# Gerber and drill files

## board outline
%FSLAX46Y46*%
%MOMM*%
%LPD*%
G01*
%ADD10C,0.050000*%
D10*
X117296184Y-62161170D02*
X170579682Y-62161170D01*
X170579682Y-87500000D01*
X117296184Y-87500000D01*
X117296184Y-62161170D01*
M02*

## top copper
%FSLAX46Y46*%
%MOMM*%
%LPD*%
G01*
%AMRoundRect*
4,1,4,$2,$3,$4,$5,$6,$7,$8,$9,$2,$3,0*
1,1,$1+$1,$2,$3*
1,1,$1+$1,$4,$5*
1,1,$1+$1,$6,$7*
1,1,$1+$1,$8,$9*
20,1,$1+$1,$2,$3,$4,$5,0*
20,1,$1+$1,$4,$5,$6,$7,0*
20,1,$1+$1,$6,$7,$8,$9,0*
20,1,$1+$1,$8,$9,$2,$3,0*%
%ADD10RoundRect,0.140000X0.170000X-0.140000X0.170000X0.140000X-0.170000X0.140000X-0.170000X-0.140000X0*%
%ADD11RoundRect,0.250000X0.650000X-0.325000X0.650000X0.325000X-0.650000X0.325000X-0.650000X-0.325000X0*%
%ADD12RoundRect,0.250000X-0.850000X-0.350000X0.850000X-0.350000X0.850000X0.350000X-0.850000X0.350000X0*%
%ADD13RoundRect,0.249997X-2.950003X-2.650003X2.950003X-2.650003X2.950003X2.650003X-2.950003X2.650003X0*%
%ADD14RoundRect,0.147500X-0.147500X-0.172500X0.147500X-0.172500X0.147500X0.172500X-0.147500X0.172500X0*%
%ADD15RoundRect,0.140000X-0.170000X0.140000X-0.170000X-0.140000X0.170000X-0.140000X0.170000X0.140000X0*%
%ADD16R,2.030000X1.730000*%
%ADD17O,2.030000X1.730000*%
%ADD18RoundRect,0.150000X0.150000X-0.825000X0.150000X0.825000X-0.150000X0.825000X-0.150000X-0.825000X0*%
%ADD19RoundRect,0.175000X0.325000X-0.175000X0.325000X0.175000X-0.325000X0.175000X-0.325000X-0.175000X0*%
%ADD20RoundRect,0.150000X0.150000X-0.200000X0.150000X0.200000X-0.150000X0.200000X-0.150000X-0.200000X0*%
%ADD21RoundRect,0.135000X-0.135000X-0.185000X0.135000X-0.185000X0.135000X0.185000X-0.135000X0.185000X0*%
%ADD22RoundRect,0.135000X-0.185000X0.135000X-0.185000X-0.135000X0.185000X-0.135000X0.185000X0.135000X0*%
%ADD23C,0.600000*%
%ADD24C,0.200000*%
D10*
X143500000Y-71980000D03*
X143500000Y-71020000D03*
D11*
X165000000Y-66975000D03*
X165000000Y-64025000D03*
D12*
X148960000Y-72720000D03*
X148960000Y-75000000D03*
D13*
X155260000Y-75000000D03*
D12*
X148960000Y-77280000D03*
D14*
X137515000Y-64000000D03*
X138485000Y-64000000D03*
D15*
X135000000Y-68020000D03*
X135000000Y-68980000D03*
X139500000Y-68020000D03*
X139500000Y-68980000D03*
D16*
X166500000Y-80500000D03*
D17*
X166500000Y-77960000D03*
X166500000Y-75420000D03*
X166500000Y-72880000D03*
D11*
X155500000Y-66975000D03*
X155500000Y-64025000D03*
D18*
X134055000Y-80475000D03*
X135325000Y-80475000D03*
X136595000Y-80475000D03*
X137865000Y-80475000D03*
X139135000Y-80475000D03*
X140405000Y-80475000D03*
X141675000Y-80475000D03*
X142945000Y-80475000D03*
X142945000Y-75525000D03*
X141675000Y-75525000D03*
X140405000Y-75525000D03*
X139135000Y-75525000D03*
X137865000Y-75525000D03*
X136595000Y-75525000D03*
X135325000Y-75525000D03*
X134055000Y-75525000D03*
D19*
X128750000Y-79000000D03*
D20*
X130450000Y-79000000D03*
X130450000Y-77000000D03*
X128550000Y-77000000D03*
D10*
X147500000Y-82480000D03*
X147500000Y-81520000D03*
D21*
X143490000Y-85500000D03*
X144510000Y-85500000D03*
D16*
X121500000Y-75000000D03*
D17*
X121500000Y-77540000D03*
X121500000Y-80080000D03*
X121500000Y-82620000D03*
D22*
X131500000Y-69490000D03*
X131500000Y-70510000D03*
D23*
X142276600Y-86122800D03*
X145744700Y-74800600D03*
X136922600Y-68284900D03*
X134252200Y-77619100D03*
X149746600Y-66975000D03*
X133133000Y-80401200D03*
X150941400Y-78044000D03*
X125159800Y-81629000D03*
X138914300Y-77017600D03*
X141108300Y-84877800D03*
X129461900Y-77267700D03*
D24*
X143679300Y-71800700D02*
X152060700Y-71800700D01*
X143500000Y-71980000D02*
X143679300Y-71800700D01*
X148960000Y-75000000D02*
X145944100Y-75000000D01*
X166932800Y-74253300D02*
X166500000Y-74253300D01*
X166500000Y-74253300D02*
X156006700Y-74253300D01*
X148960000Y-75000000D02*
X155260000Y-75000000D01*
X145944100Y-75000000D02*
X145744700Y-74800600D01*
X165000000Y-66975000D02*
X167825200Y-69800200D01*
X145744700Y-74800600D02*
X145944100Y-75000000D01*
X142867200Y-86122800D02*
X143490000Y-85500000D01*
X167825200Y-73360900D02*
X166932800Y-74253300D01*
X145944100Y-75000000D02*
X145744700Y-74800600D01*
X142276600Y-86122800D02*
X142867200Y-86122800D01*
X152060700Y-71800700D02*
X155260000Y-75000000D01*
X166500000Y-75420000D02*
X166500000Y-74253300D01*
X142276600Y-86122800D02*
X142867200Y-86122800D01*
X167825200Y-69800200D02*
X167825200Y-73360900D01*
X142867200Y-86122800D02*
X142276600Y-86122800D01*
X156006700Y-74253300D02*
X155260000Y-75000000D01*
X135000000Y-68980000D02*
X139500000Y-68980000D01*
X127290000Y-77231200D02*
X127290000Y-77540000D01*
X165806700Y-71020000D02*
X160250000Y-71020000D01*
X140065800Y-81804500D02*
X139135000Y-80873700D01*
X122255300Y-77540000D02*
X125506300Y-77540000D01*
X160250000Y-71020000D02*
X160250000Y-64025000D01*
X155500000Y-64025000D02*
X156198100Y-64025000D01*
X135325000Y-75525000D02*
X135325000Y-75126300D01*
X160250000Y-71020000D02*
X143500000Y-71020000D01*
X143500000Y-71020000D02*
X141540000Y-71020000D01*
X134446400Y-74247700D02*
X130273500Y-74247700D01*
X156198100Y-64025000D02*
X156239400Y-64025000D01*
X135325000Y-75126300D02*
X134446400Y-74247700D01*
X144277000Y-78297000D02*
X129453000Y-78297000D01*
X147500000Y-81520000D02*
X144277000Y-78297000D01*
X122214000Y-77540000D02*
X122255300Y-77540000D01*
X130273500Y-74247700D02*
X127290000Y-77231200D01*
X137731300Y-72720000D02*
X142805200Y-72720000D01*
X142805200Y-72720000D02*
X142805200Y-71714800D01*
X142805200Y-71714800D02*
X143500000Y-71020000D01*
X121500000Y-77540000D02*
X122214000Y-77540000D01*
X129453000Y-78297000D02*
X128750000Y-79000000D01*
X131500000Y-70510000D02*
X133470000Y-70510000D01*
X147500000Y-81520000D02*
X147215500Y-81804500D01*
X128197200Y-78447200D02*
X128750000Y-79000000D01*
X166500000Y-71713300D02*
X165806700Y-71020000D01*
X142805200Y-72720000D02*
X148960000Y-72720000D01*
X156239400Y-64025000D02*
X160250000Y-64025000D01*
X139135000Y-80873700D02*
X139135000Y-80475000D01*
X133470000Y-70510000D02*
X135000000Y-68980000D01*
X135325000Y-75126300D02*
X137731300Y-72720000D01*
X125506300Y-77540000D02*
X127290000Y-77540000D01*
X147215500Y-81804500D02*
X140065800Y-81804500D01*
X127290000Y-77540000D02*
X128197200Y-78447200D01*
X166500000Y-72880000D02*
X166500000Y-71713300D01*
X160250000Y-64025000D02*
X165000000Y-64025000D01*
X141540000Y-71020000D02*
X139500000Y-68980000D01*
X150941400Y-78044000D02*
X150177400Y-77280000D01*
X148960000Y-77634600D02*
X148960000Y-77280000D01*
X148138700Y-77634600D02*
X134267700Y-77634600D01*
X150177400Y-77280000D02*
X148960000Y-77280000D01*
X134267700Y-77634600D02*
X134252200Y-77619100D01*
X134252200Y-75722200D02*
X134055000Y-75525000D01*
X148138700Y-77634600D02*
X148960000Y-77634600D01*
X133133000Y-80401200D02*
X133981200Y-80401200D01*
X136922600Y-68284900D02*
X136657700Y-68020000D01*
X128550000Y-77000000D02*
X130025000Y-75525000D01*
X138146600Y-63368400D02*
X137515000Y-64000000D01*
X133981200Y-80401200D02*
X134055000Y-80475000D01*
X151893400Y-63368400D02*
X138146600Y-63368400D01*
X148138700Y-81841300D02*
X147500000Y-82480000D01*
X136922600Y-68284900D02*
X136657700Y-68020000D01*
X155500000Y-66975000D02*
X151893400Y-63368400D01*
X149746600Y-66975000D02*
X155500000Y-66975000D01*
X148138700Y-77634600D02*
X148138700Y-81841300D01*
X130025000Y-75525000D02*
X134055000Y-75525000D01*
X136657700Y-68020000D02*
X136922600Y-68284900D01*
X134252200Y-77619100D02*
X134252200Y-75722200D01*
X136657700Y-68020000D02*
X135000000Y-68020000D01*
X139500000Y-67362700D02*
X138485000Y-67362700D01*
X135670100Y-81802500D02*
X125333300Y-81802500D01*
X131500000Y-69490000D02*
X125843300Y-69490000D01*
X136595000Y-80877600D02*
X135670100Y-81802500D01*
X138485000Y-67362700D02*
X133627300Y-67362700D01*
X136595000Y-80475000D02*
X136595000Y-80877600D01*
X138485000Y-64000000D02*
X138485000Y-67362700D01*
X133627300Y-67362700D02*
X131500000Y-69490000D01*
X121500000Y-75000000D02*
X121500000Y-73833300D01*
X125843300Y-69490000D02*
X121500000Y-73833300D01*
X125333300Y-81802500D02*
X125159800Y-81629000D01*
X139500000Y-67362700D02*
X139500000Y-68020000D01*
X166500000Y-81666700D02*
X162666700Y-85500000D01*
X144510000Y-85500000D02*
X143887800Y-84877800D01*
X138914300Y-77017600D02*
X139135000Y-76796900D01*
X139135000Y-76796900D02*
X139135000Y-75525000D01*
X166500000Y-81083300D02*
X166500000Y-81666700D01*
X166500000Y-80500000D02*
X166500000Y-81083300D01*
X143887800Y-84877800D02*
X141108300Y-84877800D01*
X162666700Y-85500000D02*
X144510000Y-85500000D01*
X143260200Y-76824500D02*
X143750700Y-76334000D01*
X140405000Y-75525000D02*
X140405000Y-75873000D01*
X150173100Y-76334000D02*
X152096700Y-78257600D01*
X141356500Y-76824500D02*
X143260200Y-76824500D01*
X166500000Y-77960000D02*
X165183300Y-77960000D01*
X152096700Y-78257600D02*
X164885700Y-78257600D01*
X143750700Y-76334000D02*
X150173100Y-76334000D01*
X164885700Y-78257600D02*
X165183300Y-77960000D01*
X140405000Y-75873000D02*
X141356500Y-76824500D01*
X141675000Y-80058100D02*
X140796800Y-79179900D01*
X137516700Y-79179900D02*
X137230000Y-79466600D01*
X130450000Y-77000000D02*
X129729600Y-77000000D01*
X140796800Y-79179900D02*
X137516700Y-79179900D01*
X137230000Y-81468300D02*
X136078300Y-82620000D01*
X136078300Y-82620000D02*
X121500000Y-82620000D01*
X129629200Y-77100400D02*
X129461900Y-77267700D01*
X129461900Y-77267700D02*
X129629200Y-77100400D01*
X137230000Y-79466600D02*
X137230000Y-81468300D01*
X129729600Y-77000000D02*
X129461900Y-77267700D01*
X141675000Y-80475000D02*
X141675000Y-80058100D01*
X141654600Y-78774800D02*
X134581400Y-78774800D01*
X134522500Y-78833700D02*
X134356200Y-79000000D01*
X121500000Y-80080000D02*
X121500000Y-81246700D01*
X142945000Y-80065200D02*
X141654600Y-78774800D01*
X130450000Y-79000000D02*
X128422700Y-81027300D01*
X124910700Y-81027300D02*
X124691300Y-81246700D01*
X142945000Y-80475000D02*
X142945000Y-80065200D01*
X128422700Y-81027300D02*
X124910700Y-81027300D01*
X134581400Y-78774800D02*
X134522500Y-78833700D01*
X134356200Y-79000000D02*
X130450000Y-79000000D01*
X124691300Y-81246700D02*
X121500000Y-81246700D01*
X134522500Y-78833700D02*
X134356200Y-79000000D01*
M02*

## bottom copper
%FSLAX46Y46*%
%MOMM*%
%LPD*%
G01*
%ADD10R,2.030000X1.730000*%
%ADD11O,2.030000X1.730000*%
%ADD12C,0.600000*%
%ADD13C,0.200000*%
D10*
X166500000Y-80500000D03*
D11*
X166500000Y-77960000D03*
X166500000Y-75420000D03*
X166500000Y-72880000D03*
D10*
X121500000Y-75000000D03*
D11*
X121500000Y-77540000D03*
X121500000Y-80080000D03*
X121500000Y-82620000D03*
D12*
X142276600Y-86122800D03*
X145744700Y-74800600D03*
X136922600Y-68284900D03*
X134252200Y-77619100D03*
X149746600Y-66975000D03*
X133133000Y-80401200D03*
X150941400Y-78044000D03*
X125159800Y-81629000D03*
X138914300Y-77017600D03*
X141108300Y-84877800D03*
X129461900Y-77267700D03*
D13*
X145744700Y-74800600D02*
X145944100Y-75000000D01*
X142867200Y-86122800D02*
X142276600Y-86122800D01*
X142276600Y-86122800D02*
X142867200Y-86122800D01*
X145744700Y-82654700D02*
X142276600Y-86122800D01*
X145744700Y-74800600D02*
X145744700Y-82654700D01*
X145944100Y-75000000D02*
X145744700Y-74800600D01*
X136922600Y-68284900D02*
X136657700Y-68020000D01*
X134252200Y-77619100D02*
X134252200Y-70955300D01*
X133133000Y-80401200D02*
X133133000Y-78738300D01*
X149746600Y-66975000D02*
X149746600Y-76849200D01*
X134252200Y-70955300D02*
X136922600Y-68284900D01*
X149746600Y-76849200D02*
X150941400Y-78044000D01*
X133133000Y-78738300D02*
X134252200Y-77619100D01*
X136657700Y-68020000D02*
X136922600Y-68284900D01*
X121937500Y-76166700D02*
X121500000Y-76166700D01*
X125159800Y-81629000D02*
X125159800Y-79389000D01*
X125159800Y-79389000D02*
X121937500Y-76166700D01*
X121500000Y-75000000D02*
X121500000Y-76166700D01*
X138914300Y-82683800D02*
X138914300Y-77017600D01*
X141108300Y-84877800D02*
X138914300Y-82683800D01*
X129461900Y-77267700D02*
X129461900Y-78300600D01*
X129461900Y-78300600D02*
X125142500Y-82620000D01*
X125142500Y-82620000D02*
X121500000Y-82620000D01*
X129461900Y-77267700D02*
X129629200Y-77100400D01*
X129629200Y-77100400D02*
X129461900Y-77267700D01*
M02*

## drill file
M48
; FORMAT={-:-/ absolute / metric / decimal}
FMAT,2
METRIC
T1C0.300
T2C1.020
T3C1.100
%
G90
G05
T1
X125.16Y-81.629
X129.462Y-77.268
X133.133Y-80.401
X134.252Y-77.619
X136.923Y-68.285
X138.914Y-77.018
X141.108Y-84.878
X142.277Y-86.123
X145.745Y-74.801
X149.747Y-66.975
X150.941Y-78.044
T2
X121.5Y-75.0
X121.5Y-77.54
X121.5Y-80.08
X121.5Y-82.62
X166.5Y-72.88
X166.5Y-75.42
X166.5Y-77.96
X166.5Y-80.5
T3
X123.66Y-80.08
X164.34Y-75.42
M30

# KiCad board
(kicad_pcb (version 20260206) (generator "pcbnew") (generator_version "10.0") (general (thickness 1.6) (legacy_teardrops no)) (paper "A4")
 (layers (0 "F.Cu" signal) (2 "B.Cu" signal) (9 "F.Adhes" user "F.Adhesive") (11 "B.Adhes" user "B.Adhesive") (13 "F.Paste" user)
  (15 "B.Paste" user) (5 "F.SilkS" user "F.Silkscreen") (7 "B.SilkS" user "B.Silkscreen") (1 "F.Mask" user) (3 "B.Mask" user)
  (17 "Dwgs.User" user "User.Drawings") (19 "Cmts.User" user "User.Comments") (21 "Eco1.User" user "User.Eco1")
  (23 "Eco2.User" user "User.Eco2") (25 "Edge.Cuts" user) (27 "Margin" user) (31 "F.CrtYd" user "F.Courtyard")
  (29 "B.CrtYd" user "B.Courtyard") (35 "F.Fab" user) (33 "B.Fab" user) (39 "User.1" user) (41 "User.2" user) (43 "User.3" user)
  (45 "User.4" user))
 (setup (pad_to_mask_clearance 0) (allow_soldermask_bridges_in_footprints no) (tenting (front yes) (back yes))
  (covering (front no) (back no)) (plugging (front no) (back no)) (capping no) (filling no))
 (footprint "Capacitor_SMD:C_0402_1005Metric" (layer "F.Cu") (at 143.5 71.5 90)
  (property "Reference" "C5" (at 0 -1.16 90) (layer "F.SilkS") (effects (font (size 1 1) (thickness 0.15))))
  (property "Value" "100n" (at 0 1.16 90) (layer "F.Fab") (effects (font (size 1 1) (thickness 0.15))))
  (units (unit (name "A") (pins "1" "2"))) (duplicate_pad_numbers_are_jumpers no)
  (pad "1" smd roundrect (at -0.48 0 90) (size 0.56 0.62) (layers "F.Cu" "F.Mask" "F.Paste") (roundrect_rratio 0.25) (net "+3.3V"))
  (pad "2" smd roundrect (at 0.48 0 90) (size 0.56 0.62) (layers "F.Cu" "F.Mask" "F.Paste") (roundrect_rratio 0.25) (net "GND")))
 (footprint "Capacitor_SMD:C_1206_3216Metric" (layer "F.Cu") (at 165 65.5 90)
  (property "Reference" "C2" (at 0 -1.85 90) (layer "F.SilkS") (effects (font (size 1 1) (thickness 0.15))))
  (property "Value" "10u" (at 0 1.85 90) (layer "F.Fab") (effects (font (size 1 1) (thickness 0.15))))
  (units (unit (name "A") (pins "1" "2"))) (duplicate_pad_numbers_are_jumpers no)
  (pad "1" smd roundrect (at -1.475 0 90) (size 1.15 1.8) (layers "F.Cu" "F.Mask" "F.Paste") (roundrect_rratio 0.217391) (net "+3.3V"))
  (pad "2" smd roundrect (at 1.475 0 90) (size 1.15 1.8) (layers "F.Cu" "F.Mask" "F.Paste") (roundrect_rratio 0.217391) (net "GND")))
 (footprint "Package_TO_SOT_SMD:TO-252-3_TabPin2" (layer "F.Cu") (at 154 75)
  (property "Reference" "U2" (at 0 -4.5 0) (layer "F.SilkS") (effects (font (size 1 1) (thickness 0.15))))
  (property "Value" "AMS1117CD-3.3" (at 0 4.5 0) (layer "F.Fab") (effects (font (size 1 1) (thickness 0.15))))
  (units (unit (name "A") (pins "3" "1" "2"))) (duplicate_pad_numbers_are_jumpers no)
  (pad "" smd roundrect (at -0.415 -1.525) (size 3.05 2.75) (layers "F.Paste") (roundrect_rratio 0.090909))
  (pad "" smd roundrect (at -0.415 1.525) (size 3.05 2.75) (layers "F.Paste") (roundrect_rratio 0.090909))
  (pad "" smd roundrect (at 2.935 -1.525) (size 3.05 2.75) (layers "F.Paste") (roundrect_rratio 0.090909))
  (pad "" smd roundrect (at 2.935 1.525) (size 3.05 2.75) (layers "F.Paste") (roundrect_rratio 0.090909))
  (pad "1" smd roundrect (at -5.04 -2.28) (size 2.2 1.2) (layers "F.Cu" "F.Mask" "F.Paste") (roundrect_rratio 0.208333) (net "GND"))
  (pad "2" smd roundrect (at -5.04 0) (size 2.2 1.2) (layers "F.Cu" "F.Mask" "F.Paste") (roundrect_rratio 0.208333) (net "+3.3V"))
  (pad "2" smd roundrect (at 1.26 0) (size 6.4 5.8) (layers "F.Cu" "F.Mask") (roundrect_rratio 0.043103) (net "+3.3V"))
  (pad "3" smd roundrect (at -5.04 2.28) (size 2.2 1.2) (layers "F.Cu" "F.Mask" "F.Paste") (roundrect_rratio 0.208333) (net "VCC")))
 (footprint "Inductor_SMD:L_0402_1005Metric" (layer "F.Cu") (at 138 64)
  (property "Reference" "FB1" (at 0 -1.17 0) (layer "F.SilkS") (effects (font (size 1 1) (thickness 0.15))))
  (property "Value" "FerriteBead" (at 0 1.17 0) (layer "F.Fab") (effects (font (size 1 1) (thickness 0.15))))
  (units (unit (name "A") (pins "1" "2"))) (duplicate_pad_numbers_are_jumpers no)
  (pad "1" smd roundrect (at -0.485 0) (size 0.59 0.64) (layers "F.Cu" "F.Mask" "F.Paste") (roundrect_rratio 0.25) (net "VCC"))
  (pad "2" smd roundrect (at 0.485 0) (size 0.59 0.64) (layers "F.Cu" "F.Mask" "F.Paste") (roundrect_rratio 0.25) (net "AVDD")))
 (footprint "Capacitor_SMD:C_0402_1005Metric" (layer "F.Cu") (at 135 68.5 -90)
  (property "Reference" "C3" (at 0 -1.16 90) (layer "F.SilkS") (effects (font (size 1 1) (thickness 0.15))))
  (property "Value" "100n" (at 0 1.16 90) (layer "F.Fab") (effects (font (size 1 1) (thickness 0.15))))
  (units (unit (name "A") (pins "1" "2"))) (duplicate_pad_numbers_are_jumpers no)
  (pad "1" smd roundrect (at -0.48 0 270) (size 0.56 0.62) (layers "F.Cu" "F.Mask" "F.Paste") (roundrect_rratio 0.25) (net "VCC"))
  (pad "2" smd roundrect (at 0.48 0 270) (size 0.56 0.62) (layers "F.Cu" "F.Mask" "F.Paste") (roundrect_rratio 0.25) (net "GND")))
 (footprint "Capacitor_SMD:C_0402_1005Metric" (layer "F.Cu") (at 139.5 68.5 -90)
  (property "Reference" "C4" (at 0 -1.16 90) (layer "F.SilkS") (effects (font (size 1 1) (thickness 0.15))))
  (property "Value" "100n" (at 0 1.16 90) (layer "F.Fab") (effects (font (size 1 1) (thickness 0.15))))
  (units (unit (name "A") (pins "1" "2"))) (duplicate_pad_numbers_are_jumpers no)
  (pad "1" smd roundrect (at -0.48 0 270) (size 0.56 0.62) (layers "F.Cu" "F.Mask" "F.Paste") (roundrect_rratio 0.25) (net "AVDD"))
  (pad "2" smd roundrect (at 0.48 0 270) (size 0.56 0.62) (layers "F.Cu" "F.Mask" "F.Paste") (roundrect_rratio 0.25) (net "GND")))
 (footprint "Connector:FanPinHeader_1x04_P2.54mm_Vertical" (layer "F.Cu") (at 166.5 80.5 90)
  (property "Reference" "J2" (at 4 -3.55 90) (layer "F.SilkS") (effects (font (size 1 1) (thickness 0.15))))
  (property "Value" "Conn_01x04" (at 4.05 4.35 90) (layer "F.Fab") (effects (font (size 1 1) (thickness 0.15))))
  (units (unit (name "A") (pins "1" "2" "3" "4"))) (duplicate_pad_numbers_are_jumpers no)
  (pad "" np_thru_hole circle (at 5.08 -2.16 180) (size 1.1 1.1) (drill 1.1) (layers "*.Cu" "*.Mask"))
  (pad "1" thru_hole rect (at 0 0 180) (size 2.03 1.73) (drill 1.02) (layers "*.Cu" "*.Mask") (remove_unused_layers no) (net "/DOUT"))
  (pad "2" thru_hole oval (at 2.54 0 180) (size 2.03 1.73) (drill 1.02) (layers "*.Cu" "*.Mask") (remove_unused_layers no) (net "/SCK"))
  (pad "3" thru_hole oval (at 5.08 0 180) (size 2.03 1.73) (drill 1.02) (layers "*.Cu" "*.Mask") (remove_unused_layers no) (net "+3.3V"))
  (pad "4" thru_hole oval (at 7.62 0 180) (size 2.03 1.73) (drill 1.02) (layers "*.Cu" "*.Mask") (remove_unused_layers no) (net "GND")))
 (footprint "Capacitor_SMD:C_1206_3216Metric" (layer "F.Cu") (at 155.5 65.5 90)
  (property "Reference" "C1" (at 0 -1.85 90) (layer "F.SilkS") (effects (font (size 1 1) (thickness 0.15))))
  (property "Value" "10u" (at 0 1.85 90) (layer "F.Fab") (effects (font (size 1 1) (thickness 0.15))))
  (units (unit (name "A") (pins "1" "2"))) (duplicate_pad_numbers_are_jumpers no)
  (pad "1" smd roundrect (at -1.475 0 90) (size 1.15 1.8) (layers "F.Cu" "F.Mask" "F.Paste") (roundrect_rratio 0.217391) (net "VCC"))
  (pad "2" smd roundrect (at 1.475 0 90) (size 1.15 1.8) (layers "F.Cu" "F.Mask" "F.Paste") (roundrect_rratio 0.217391) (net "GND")))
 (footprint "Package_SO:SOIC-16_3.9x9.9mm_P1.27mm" (layer "F.Cu") (at 138.5 78 90)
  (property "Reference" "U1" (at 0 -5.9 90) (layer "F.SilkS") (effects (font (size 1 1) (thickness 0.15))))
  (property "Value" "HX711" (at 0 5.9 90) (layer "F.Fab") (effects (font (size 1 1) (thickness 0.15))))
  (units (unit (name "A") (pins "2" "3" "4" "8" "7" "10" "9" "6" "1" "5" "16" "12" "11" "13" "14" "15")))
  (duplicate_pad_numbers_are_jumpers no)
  (pad "1" smd roundrect (at -2.475 -4.445 90) (size 1.95 0.6) (layers "F.Cu" "F.Mask" "F.Paste") (roundrect_rratio 0.25) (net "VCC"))
  (pad "2" smd roundrect (at -2.475 -3.175 90) (size 1.95 0.6) (layers "F.Cu" "F.Mask" "F.Paste") (roundrect_rratio 0.25)
   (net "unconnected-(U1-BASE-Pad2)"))
  (pad "3" smd roundrect (at -2.475 -1.905 90) (size 1.95 0.6) (layers "F.Cu" "F.Mask" "F.Paste") (roundrect_rratio 0.25) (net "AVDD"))
  (pad "4" smd roundrect (at -2.475 -0.635 90) (size 1.95 0.6) (layers "F.Cu" "F.Mask" "F.Paste") (roundrect_rratio 0.25)
   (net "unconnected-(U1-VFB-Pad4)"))
  (pad "5" smd roundrect (at -2.475 0.635 90) (size 1.95 0.6) (layers "F.Cu" "F.Mask" "F.Paste") (roundrect_rratio 0.25) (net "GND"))
  (pad "6" smd roundrect (at -2.475 1.905 90) (size 1.95 0.6) (layers "F.Cu" "F.Mask" "F.Paste") (roundrect_rratio 0.25)
   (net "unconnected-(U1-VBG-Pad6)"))
  (pad "7" smd roundrect (at -2.475 3.175 90) (size 1.95 0.6) (layers "F.Cu" "F.Mask" "F.Paste") (roundrect_rratio 0.25) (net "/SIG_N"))
  (pad "8" smd roundrect (at -2.475 4.445 90) (size 1.95 0.6) (layers "F.Cu" "F.Mask" "F.Paste") (roundrect_rratio 0.25) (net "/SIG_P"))
  (pad "9" smd roundrect (at 2.475 4.445 90) (size 1.95 0.6) (layers "F.Cu" "F.Mask" "F.Paste") (roundrect_rratio 0.25)
   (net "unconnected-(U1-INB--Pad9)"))
  (pad "10" smd roundrect (at 2.475 3.175 90) (size 1.95 0.6) (layers "F.Cu" "F.Mask" "F.Paste") (roundrect_rratio 0.25)
   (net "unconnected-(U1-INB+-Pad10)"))
  (pad "11" smd roundrect (at 2.475 1.905 90) (size 1.95 0.6) (layers "F.Cu" "F.Mask" "F.Paste") (roundrect_rratio 0.25) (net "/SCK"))
  (pad "12" smd roundrect (at 2.475 0.635 90) (size 1.95 0.6) (layers "F.Cu" "F.Mask" "F.Paste") (roundrect_rratio 0.25) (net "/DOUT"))
  (pad "13" smd roundrect (at 2.475 -0.635 90) (size 1.95 0.6) (layers "F.Cu" "F.Mask" "F.Paste") (roundrect_rratio 0.25)
   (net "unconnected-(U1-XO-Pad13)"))
  (pad "14" smd roundrect (at 2.475 -1.905 90) (size 1.95 0.6) (layers "F.Cu" "F.Mask" "F.Paste") (roundrect_rratio 0.25)
   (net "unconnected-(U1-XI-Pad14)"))
  (pad "15" smd roundrect (at 2.475 -3.175 90) (size 1.95 0.6) (layers "F.Cu" "F.Mask" "F.Paste") (roundrect_rratio 0.25) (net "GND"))
  (pad "16" smd roundrect (at 2.475 -4.445 90) (size 1.95 0.6) (layers "F.Cu" "F.Mask" "F.Paste") (roundrect_rratio 0.25) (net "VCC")))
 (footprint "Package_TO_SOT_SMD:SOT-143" (layer "F.Cu") (at 129.5 78 90)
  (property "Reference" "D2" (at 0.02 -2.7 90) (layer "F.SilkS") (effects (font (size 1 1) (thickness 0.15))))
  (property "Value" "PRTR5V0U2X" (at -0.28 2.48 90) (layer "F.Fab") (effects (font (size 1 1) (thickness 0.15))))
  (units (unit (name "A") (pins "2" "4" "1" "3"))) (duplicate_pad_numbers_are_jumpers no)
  (pad "1" smd roundrect (at -1 -0.75 90) (size 0.7 1) (layers "F.Cu" "F.Mask" "F.Paste") (roundrect_rratio 0.25) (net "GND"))
  (pad "2" smd roundrect (at -1 0.95 90) (size 0.7 0.6) (layers "F.Cu" "F.Mask" "F.Paste") (roundrect_rratio 0.25) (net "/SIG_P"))
  (pad "3" smd roundrect (at 1 0.95 90) (size 0.7 0.6) (layers "F.Cu" "F.Mask" "F.Paste") (roundrect_rratio 0.25) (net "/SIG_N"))
  (pad "4" smd roundrect (at 1 -0.95 90) (size 0.7 0.6) (layers "F.Cu" "F.Mask" "F.Paste") (roundrect_rratio 0.25) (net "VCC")))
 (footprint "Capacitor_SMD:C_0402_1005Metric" (layer "F.Cu") (at 147.5 82 90)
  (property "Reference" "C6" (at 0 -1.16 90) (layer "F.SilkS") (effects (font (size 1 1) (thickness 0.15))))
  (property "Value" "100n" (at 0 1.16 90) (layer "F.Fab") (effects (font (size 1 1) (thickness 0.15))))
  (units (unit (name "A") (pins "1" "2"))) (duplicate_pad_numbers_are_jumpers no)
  (pad "1" smd roundrect (at -0.48 0 90) (size 0.56 0.62) (layers "F.Cu" "F.Mask" "F.Paste") (roundrect_rratio 0.25) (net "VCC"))
  (pad "2" smd roundrect (at 0.48 0 90) (size 0.56 0.62) (layers "F.Cu" "F.Mask" "F.Paste") (roundrect_rratio 0.25) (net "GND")))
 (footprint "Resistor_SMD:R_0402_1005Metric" (layer "F.Cu") (at 144 85.5)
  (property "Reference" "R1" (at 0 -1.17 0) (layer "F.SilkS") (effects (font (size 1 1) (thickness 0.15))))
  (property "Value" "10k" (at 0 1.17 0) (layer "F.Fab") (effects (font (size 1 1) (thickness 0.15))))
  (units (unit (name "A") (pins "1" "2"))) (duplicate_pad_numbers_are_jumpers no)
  (pad "1" smd roundrect (at -0.51 0) (size 0.54 0.64) (layers "F.Cu" "F.Mask" "F.Paste") (roundrect_rratio 0.25) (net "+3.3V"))
  (pad "2" smd roundrect (at 0.51 0) (size 0.54 0.64) (layers "F.Cu" "F.Mask" "F.Paste") (roundrect_rratio 0.25) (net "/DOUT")))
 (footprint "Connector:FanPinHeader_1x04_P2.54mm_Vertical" (layer "F.Cu") (at 121.5 75 -90)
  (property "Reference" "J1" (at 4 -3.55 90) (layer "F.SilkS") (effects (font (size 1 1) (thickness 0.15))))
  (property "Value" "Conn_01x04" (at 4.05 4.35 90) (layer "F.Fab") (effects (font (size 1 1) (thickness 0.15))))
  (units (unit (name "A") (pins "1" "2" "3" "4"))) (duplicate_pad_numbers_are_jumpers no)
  (pad "" np_thru_hole circle (at 5.08 -2.16) (size 1.1 1.1) (drill 1.1) (layers "*.Cu" "*.Mask"))
  (pad "1" thru_hole rect (at 0 0) (size 2.03 1.73) (drill 1.02) (layers "*.Cu" "*.Mask") (remove_unused_layers no) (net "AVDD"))
  (pad "2" thru_hole oval (at 2.54 0) (size 2.03 1.73) (drill 1.02) (layers "*.Cu" "*.Mask") (remove_unused_layers no) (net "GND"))
  (pad "3" thru_hole oval (at 5.08 0) (size 2.03 1.73) (drill 1.02) (layers "*.Cu" "*.Mask") (remove_unused_layers no) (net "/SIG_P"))
  (pad "4" thru_hole oval (at 7.62 0) (size 2.03 1.73) (drill 1.02) (layers "*.Cu" "*.Mask") (remove_unused_layers no) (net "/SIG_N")))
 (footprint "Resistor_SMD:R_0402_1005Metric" (layer "F.Cu") (at 131.5 70 -90)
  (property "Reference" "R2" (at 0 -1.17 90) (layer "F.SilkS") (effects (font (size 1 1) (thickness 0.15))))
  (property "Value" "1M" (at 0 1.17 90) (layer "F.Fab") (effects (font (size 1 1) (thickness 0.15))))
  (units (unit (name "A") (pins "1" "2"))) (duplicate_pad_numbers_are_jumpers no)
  (pad "1" smd roundrect (at -0.51 0 270) (size 0.54 0.64) (layers "F.Cu" "F.Mask" "F.Paste") (roundrect_rratio 0.25) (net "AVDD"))
  (pad "2" smd roundrect (at 0.51 0 270) (size 0.54 0.64) (layers "F.Cu" "F.Mask" "F.Paste") (roundrect_rratio 0.25) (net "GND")))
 (gr_rect (start 117.296184 62.16117) (end 170.579682 87.5) (stroke (width 0.05) (type default)) (fill no) (layer "Edge.Cuts"))
 (segment (start 143.6793 71.8007) (end 152.0607 71.8007) (width 0.2) (layer "F.Cu") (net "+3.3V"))
 (segment (start 143.5 71.98) (end 143.6793 71.8007) (width 0.2) (layer "F.Cu") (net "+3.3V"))
 (segment (start 148.96 75) (end 145.9441 75) (width 0.2) (layer "F.Cu") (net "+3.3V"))
 (segment (start 166.9328 74.2533) (end 166.5 74.2533) (width 0.2) (layer "F.Cu") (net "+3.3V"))
 (segment (start 166.5 74.2533) (end 156.0067 74.2533) (width 0.2) (layer "F.Cu") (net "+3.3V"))
 (segment (start 148.96 75) (end 155.26 75) (width 0.2) (layer "F.Cu") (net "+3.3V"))
 (segment (start 145.9441 75) (end 145.7447 74.8006) (width 0.2) (layer "F.Cu") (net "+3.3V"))
 (segment (start 165 66.975) (end 167.8252 69.8002) (width 0.2) (layer "F.Cu") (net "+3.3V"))
 (segment (start 145.7447 74.8006) (end 145.9441 75) (width 0.2) (layer "F.Cu") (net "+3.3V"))
 (segment (start 142.8672 86.1228) (end 143.49 85.5) (width 0.2) (layer "F.Cu") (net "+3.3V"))
 (segment (start 167.8252 73.3609) (end 166.9328 74.2533) (width 0.2) (layer "F.Cu") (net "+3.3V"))
 (segment (start 145.9441 75) (end 145.7447 74.8006) (width 0.2) (layer "F.Cu") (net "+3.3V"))
 (segment (start 142.2766 86.1228) (end 142.8672 86.1228) (width 0.2) (layer "F.Cu") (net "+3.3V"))
 (segment (start 152.0607 71.8007) (end 155.26 75) (width 0.2) (layer "F.Cu") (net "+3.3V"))
 (segment (start 166.5 75.42) (end 166.5 74.2533) (width 0.2) (layer "F.Cu") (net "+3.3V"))
 (segment (start 142.2766 86.1228) (end 142.8672 86.1228) (width 0.2) (layer "F.Cu") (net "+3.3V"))
 (segment (start 167.8252 69.8002) (end 167.8252 73.3609) (width 0.2) (layer "F.Cu") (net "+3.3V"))
 (segment (start 142.8672 86.1228) (end 142.2766 86.1228) (width 0.2) (layer "F.Cu") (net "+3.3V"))
 (segment (start 156.0067 74.2533) (end 155.26 75) (width 0.2) (layer "F.Cu") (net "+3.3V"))
 (via (at 142.2766 86.1228) (size 0.6) (drill 0.3) (layers "F.Cu" "B.Cu") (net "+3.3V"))
 (via (at 145.7447 74.8006) (size 0.6) (drill 0.3) (layers "F.Cu" "B.Cu") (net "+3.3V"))
 (segment (start 145.7447 74.8006) (end 145.9441 75) (width 0.2) (layer "B.Cu") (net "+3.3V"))
 (segment (start 142.8672 86.1228) (end 142.2766 86.1228) (width 0.2) (layer "B.Cu") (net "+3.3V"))
 (segment (start 142.2766 86.1228) (end 142.8672 86.1228) (width 0.2) (layer "B.Cu") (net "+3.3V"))
 (segment (start 145.7447 82.6547) (end 142.2766 86.1228) (width 0.2) (layer "B.Cu") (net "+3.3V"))
 (segment (start 145.7447 74.8006) (end 145.7447 82.6547) (width 0.2) (layer "B.Cu") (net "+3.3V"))
 (segment (start 145.9441 75) (end 145.7447 74.8006) (width 0.2) (layer "B.Cu") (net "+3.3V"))
 (segment (start 135 68.98) (end 139.5 68.98) (width 0.2) (layer "F.Cu") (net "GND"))
 (segment (start 127.29 77.2312) (end 127.29 77.54) (width 0.2) (layer "F.Cu") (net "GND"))
 (segment (start 165.8067 71.02) (end 160.25 71.02) (width 0.2) (layer "F.Cu") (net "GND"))
 (segment (start 140.0658 81.8045) (end 139.135 80.8737) (width 0.2) (layer "F.Cu") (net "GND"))
 (segment (start 122.2553 77.54) (end 125.5063 77.54) (width 0.2) (layer "F.Cu") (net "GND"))
 (segment (start 160.25 71.02) (end 160.25 64.025) (width 0.2) (layer "F.Cu") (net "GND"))
 (segment (start 155.5 64.025) (end 156.1981 64.025) (width 0.2) (layer "F.Cu") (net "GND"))
 (segment (start 135.325 75.525) (end 135.325 75.1263) (width 0.2) (layer "F.Cu") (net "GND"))
 (segment (start 160.25 71.02) (end 143.5 71.02) (width 0.2) (layer "F.Cu") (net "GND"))
 (segment (start 143.5 71.02) (end 141.54 71.02) (width 0.2) (layer "F.Cu") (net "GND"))
 (segment (start 134.4464 74.2477) (end 130.2735 74.2477) (width 0.2) (layer "F.Cu") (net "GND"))
 (segment (start 156.1981 64.025) (end 156.2394 64.025) (width 0.2) (layer "F.Cu") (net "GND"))
 (segment (start 135.325 75.1263) (end 134.4464 74.2477) (width 0.2) (layer "F.Cu") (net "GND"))
 (segment (start 144.277 78.297) (end 129.453 78.297) (width 0.2) (layer "F.Cu") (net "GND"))
 (segment (start 147.5 81.52) (end 144.277 78.297) (width 0.2) (layer "F.Cu") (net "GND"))
 (segment (start 122.214 77.54) (end 122.2553 77.54) (width 0.2) (layer "F.Cu") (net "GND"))
 (segment (start 130.2735 74.2477) (end 127.29 77.2312) (width 0.2) (layer "F.Cu") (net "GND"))
 (segment (start 137.7313 72.72) (end 142.8052 72.72) (width 0.2) (layer "F.Cu") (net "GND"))
 (segment (start 142.8052 72.72) (end 142.8052 71.7148) (width 0.2) (layer "F.Cu") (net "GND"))
 (segment (start 142.8052 71.7148) (end 143.5 71.02) (width 0.2) (layer "F.Cu") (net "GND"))
 (segment (start 121.5 77.54) (end 122.214 77.54) (width 0.2) (layer "F.Cu") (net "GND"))
 (segment (start 129.453 78.297) (end 128.75 79) (width 0.2) (layer "F.Cu") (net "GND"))
 (segment (start 131.5 70.51) (end 133.47 70.51) (width 0.2) (layer "F.Cu") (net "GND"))
 (segment (start 147.5 81.52) (end 147.2155 81.8045) (width 0.2) (layer "F.Cu") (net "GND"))
 (segment (start 128.1972 78.4472) (end 128.75 79) (width 0.2) (layer "F.Cu") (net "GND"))
 (segment (start 166.5 71.7133) (end 165.8067 71.02) (width 0.2) (layer "F.Cu") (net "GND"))
 (segment (start 142.8052 72.72) (end 148.96 72.72) (width 0.2) (layer "F.Cu") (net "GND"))
 (segment (start 156.2394 64.025) (end 160.25 64.025) (width 0.2) (layer "F.Cu") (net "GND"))
 (segment (start 139.135 80.8737) (end 139.135 80.475) (width 0.2) (layer "F.Cu") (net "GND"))
 (segment (start 133.47 70.51) (end 135 68.98) (width 0.2) (layer "F.Cu") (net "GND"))
 (segment (start 135.325 75.1263) (end 137.7313 72.72) (width 0.2) (layer "F.Cu") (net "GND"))
 (segment (start 125.5063 77.54) (end 127.29 77.54) (width 0.2) (layer "F.Cu") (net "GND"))
 (segment (start 147.2155 81.8045) (end 140.0658 81.8045) (width 0.2) (layer "F.Cu") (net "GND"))
 (segment (start 127.29 77.54) (end 128.1972 78.4472) (width 0.2) (layer "F.Cu") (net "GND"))
 (segment (start 166.5 72.88) (end 166.5 71.7133) (width 0.2) (layer "F.Cu") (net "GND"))
 (segment (start 160.25 64.025) (end 165 64.025) (width 0.2) (layer "F.Cu") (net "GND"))
 (segment (start 141.54 71.02) (end 139.5 68.98) (width 0.2) (layer "F.Cu") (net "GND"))
 (segment (start 150.9414 78.044) (end 150.1774 77.28) (width 0.2) (layer "F.Cu") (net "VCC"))
 (segment (start 148.96 77.6346) (end 148.96 77.28) (width 0.2) (layer "F.Cu") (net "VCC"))
 (segment (start 148.1387 77.6346) (end 134.2677 77.6346) (width 0.2) (layer "F.Cu") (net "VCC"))
 (segment (start 150.1774 77.28) (end 148.96 77.28) (width 0.2) (layer "F.Cu") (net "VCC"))
 (segment (start 134.2677 77.6346) (end 134.2522 77.6191) (width 0.2) (layer "F.Cu") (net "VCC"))
 (segment (start 134.2522 75.7222) (end 134.055 75.525) (width 0.2) (layer "F.Cu") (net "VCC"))
 (segment (start 148.1387 77.6346) (end 148.96 77.6346) (width 0.2) (layer "F.Cu") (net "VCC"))
 (segment (start 133.133 80.4012) (end 133.9812 80.4012) (width 0.2) (layer "F.Cu") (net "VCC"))
 (segment (start 136.9226 68.2849) (end 136.6577 68.02) (width 0.2) (layer "F.Cu") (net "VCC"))
 (segment (start 128.55 77) (end 130.025 75.525) (width 0.2) (layer "F.Cu") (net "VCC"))
 (segment (start 138.1466 63.3684) (end 137.515 64) (width 0.2) (layer "F.Cu") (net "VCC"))
 (segment (start 133.9812 80.4012) (end 134.055 80.475) (width 0.2) (layer "F.Cu") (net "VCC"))
 (segment (start 151.8934 63.3684) (end 138.1466 63.3684) (width 0.2) (layer "F.Cu") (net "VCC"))
 (segment (start 148.1387 81.8413) (end 147.5 82.48) (width 0.2) (layer "F.Cu") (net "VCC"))
 (segment (start 136.9226 68.2849) (end 136.6577 68.02) (width 0.2) (layer "F.Cu") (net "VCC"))
 (segment (start 155.5 66.975) (end 151.8934 63.3684) (width 0.2) (layer "F.Cu") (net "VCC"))
 (segment (start 149.7466 66.975) (end 155.5 66.975) (width 0.2) (layer "F.Cu") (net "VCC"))
 (segment (start 148.1387 77.6346) (end 148.1387 81.8413) (width 0.2) (layer "F.Cu") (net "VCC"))
 (segment (start 130.025 75.525) (end 134.055 75.525) (width 0.2) (layer "F.Cu") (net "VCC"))
 (segment (start 136.6577 68.02) (end 136.9226 68.2849) (width 0.2) (layer "F.Cu") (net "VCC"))
 (segment (start 134.2522 77.6191) (end 134.2522 75.7222) (width 0.2) (layer "F.Cu") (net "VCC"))
 (segment (start 136.6577 68.02) (end 135 68.02) (width 0.2) (layer "F.Cu") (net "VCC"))
 (via (at 136.9226 68.2849) (size 0.6) (drill 0.3) (layers "F.Cu" "B.Cu") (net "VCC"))
 (via (at 134.2522 77.6191) (size 0.6) (drill 0.3) (layers "F.Cu" "B.Cu") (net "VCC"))
 (via (at 149.7466 66.975) (size 0.6) (drill 0.3) (layers "F.Cu" "B.Cu") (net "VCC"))
 (via (at 133.133 80.4012) (size 0.6) (drill 0.3) (layers "F.Cu" "B.Cu") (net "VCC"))
 (via (at 150.9414 78.044) (size 0.6) (drill 0.3) (layers "F.Cu" "B.Cu") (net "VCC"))
 (segment (start 136.9226 68.2849) (end 136.6577 68.02) (width 0.2) (layer "B.Cu") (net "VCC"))
 (segment (start 134.2522 77.6191) (end 134.2522 70.9553) (width 0.2) (layer "B.Cu") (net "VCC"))
 (segment (start 133.133 80.4012) (end 133.133 78.7383) (width 0.2) (layer "B.Cu") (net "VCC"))
 (segment (start 149.7466 66.975) (end 149.7466 76.8492) (width 0.2) (layer "B.Cu") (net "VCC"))
 (segment (start 134.2522 70.9553) (end 136.9226 68.2849) (width 0.2) (layer "B.Cu") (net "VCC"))
 (segment (start 149.7466 76.8492) (end 150.9414 78.044) (width 0.2) (layer "B.Cu") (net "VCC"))
 (segment (start 133.133 78.7383) (end 134.2522 77.6191) (width 0.2) (layer "B.Cu") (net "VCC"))
 (segment (start 136.6577 68.02) (end 136.9226 68.2849) (width 0.2) (layer "B.Cu") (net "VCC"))
 (segment (start 139.5 67.3627) (end 138.485 67.3627) (width 0.2) (layer "F.Cu") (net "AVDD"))
 (segment (start 135.6701 81.8025) (end 125.3333 81.8025) (width 0.2) (layer "F.Cu") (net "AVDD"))
 (segment (start 131.5 69.49) (end 125.8433 69.49) (width 0.2) (layer "F.Cu") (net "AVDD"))
 (segment (start 136.595 80.8776) (end 135.6701 81.8025) (width 0.2) (layer "F.Cu") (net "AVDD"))
 (segment (start 138.485 67.3627) (end 133.6273 67.3627) (width 0.2) (layer "F.Cu") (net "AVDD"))
 (segment (start 136.595 80.475) (end 136.595 80.8776) (width 0.2) (layer "F.Cu") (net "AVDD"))
 (segment (start 138.485 64) (end 138.485 67.3627) (width 0.2) (layer "F.Cu") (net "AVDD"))
 (segment (start 133.6273 67.3627) (end 131.5 69.49) (width 0.2) (layer "F.Cu") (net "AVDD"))
 (segment (start 121.5 75) (end 121.5 73.8333) (width 0.2) (layer "F.Cu") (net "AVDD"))
 (segment (start 125.8433 69.49) (end 121.5 73.8333) (width 0.2) (layer "F.Cu") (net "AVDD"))
 (segment (start 125.3333 81.8025) (end 125.1598 81.629) (width 0.2) (layer "F.Cu") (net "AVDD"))
 (segment (start 139.5 67.3627) (end 139.5 68.02) (width 0.2) (layer "F.Cu") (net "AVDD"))
 (via (at 125.1598 81.629) (size 0.6) (drill 0.3) (layers "F.Cu" "B.Cu") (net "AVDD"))
 (segment (start 121.9375 76.1667) (end 121.5 76.1667) (width 0.2) (layer "B.Cu") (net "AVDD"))
 (segment (start 125.1598 81.629) (end 125.1598 79.389) (width 0.2) (layer "B.Cu") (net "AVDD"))
 (segment (start 125.1598 79.389) (end 121.9375 76.1667) (width 0.2) (layer "B.Cu") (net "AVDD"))
 (segment (start 121.5 75) (end 121.5 76.1667) (width 0.2) (layer "B.Cu") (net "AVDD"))
 (segment (start 166.5 81.6667) (end 162.6667 85.5) (width 0.2) (layer "F.Cu") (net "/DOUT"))
 (segment (start 144.51 85.5) (end 143.8878 84.8778) (width 0.2) (layer "F.Cu") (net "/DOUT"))
 (segment (start 138.9143 77.0176) (end 139.135 76.7969) (width 0.2) (layer "F.Cu") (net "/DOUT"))
 (segment (start 139.135 76.7969) (end 139.135 75.525) (width 0.2) (layer "F.Cu") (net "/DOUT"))
 (segment (start 166.5 81.0833) (end 166.5 81.6667) (width 0.2) (layer "F.Cu") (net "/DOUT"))
 (segment (start 166.5 80.5) (end 166.5 81.0833) (width 0.2) (layer "F.Cu") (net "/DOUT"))
 (segment (start 143.8878 84.8778) (end 141.1083 84.8778) (width 0.2) (layer "F.Cu") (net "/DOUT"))
 (segment (start 162.6667 85.5) (end 144.51 85.5) (width 0.2) (layer "F.Cu") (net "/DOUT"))
 (via (at 138.9143 77.0176) (size 0.6) (drill 0.3) (layers "F.Cu" "B.Cu") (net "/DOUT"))
 (via (at 141.1083 84.8778) (size 0.6) (drill 0.3) (layers "F.Cu" "B.Cu") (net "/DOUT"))
 (segment (start 138.9143 82.6838) (end 138.9143 77.0176) (width 0.2) (layer "B.Cu") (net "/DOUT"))
 (segment (start 141.1083 84.8778) (end 138.9143 82.6838) (width 0.2) (layer "B.Cu") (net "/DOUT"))
 (segment (start 143.2602 76.8245) (end 143.7507 76.334) (width 0.2) (layer "F.Cu") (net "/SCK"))
 (segment (start 140.405 75.525) (end 140.405 75.873) (width 0.2) (layer "F.Cu") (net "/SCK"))
 (segment (start 150.1731 76.334) (end 152.0967 78.2576) (width 0.2) (layer "F.Cu") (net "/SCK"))
 (segment (start 141.3565 76.8245) (end 143.2602 76.8245) (width 0.2) (layer "F.Cu") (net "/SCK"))
 (segment (start 166.5 77.96) (end 165.1833 77.96) (width 0.2) (layer "F.Cu") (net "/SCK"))
 (segment (start 152.0967 78.2576) (end 164.8857 78.2576) (width 0.2) (layer "F.Cu") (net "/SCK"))
 (segment (start 143.7507 76.334) (end 150.1731 76.334) (width 0.2) (layer "F.Cu") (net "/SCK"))
 (segment (start 164.8857 78.2576) (end 165.1833 77.96) (width 0.2) (layer "F.Cu") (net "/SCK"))
 (segment (start 140.405 75.873) (end 141.3565 76.8245) (width 0.2) (layer "F.Cu") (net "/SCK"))
 (segment (start 141.675 80.0581) (end 140.7968 79.1799) (width 0.2) (layer "F.Cu") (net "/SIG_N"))
 (segment (start 137.5167 79.1799) (end 137.23 79.4666) (width 0.2) (layer "F.Cu") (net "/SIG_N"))
 (segment (start 130.45 77) (end 129.7296 77) (width 0.2) (layer "F.Cu") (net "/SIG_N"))
 (segment (start 140.7968 79.1799) (end 137.5167 79.1799) (width 0.2) (layer "F.Cu") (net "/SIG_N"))
 (segment (start 137.23 81.4683) (end 136.0783 82.62) (width 0.2) (layer "F.Cu") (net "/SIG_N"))
 (segment (start 136.0783 82.62) (end 121.5 82.62) (width 0.2) (layer "F.Cu") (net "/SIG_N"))
 (segment (start 129.6292 77.1004) (end 129.4619 77.2677) (width 0.2) (layer "F.Cu") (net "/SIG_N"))
 (segment (start 129.4619 77.2677) (end 129.6292 77.1004) (width 0.2) (layer "F.Cu") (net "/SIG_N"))
 (segment (start 137.23 79.4666) (end 137.23 81.4683) (width 0.2) (layer "F.Cu") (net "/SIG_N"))
 (segment (start 129.7296 77) (end 129.4619 77.2677) (width 0.2) (layer "F.Cu") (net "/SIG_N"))
 (segment (start 141.675 80.475) (end 141.675 80.0581) (width 0.2) (layer "F.Cu") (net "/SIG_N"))
 (via (at 129.4619 77.2677) (size 0.6) (drill 0.3) (layers "F.Cu" "B.Cu") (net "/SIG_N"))
 (segment (start 129.4619 77.2677) (end 129.4619 78.3006) (width 0.2) (layer "B.Cu") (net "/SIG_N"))
 (segment (start 129.4619 78.3006) (end 125.1425 82.62) (width 0.2) (layer "B.Cu") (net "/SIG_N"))
 (segment (start 125.1425 82.62) (end 121.5 82.62) (width 0.2) (layer "B.Cu") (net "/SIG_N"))
 (segment (start 129.4619 77.2677) (end 129.6292 77.1004) (width 0.2) (layer "B.Cu") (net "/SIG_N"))
 (segment (start 129.6292 77.1004) (end 129.4619 77.2677) (width 0.2) (layer "B.Cu") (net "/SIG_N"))
 (segment (start 141.6546 78.7748) (end 134.5814 78.7748) (width 0.2) (layer "F.Cu") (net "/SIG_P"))
 (segment (start 134.5225 78.8337) (end 134.3562 79) (width 0.2) (layer "F.Cu") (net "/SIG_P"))
 (segment (start 121.5 80.08) (end 121.5 81.2467) (width 0.2) (layer "F.Cu") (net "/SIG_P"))
 (segment (start 142.945 80.0652) (end 141.6546 78.7748) (width 0.2) (layer "F.Cu") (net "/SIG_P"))
 (segment (start 130.45 79) (end 128.4227 81.0273) (width 0.2) (layer "F.Cu") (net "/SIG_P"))
 (segment (start 124.9107 81.0273) (end 124.6913 81.2467) (width 0.2) (layer "F.Cu") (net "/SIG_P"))
 (segment (start 142.945 80.475) (end 142.945 80.0652) (width 0.2) (layer "F.Cu") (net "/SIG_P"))
 (segment (start 128.4227 81.0273) (end 124.9107 81.0273) (width 0.2) (layer "F.Cu") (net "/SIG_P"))
 (segment (start 134.5814 78.7748) (end 134.5225 78.8337) (width 0.2) (layer "F.Cu") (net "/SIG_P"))
 (segment (start 134.3562 79) (end 130.45 79) (width 0.2) (layer "F.Cu") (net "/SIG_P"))
 (segment (start 124.6913 81.2467) (end 121.5 81.2467) (width 0.2) (layer "F.Cu") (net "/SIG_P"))
 (segment (start 134.5225 78.8337) (end 134.3562 79) (width 0.2) (layer "F.Cu") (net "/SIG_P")))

